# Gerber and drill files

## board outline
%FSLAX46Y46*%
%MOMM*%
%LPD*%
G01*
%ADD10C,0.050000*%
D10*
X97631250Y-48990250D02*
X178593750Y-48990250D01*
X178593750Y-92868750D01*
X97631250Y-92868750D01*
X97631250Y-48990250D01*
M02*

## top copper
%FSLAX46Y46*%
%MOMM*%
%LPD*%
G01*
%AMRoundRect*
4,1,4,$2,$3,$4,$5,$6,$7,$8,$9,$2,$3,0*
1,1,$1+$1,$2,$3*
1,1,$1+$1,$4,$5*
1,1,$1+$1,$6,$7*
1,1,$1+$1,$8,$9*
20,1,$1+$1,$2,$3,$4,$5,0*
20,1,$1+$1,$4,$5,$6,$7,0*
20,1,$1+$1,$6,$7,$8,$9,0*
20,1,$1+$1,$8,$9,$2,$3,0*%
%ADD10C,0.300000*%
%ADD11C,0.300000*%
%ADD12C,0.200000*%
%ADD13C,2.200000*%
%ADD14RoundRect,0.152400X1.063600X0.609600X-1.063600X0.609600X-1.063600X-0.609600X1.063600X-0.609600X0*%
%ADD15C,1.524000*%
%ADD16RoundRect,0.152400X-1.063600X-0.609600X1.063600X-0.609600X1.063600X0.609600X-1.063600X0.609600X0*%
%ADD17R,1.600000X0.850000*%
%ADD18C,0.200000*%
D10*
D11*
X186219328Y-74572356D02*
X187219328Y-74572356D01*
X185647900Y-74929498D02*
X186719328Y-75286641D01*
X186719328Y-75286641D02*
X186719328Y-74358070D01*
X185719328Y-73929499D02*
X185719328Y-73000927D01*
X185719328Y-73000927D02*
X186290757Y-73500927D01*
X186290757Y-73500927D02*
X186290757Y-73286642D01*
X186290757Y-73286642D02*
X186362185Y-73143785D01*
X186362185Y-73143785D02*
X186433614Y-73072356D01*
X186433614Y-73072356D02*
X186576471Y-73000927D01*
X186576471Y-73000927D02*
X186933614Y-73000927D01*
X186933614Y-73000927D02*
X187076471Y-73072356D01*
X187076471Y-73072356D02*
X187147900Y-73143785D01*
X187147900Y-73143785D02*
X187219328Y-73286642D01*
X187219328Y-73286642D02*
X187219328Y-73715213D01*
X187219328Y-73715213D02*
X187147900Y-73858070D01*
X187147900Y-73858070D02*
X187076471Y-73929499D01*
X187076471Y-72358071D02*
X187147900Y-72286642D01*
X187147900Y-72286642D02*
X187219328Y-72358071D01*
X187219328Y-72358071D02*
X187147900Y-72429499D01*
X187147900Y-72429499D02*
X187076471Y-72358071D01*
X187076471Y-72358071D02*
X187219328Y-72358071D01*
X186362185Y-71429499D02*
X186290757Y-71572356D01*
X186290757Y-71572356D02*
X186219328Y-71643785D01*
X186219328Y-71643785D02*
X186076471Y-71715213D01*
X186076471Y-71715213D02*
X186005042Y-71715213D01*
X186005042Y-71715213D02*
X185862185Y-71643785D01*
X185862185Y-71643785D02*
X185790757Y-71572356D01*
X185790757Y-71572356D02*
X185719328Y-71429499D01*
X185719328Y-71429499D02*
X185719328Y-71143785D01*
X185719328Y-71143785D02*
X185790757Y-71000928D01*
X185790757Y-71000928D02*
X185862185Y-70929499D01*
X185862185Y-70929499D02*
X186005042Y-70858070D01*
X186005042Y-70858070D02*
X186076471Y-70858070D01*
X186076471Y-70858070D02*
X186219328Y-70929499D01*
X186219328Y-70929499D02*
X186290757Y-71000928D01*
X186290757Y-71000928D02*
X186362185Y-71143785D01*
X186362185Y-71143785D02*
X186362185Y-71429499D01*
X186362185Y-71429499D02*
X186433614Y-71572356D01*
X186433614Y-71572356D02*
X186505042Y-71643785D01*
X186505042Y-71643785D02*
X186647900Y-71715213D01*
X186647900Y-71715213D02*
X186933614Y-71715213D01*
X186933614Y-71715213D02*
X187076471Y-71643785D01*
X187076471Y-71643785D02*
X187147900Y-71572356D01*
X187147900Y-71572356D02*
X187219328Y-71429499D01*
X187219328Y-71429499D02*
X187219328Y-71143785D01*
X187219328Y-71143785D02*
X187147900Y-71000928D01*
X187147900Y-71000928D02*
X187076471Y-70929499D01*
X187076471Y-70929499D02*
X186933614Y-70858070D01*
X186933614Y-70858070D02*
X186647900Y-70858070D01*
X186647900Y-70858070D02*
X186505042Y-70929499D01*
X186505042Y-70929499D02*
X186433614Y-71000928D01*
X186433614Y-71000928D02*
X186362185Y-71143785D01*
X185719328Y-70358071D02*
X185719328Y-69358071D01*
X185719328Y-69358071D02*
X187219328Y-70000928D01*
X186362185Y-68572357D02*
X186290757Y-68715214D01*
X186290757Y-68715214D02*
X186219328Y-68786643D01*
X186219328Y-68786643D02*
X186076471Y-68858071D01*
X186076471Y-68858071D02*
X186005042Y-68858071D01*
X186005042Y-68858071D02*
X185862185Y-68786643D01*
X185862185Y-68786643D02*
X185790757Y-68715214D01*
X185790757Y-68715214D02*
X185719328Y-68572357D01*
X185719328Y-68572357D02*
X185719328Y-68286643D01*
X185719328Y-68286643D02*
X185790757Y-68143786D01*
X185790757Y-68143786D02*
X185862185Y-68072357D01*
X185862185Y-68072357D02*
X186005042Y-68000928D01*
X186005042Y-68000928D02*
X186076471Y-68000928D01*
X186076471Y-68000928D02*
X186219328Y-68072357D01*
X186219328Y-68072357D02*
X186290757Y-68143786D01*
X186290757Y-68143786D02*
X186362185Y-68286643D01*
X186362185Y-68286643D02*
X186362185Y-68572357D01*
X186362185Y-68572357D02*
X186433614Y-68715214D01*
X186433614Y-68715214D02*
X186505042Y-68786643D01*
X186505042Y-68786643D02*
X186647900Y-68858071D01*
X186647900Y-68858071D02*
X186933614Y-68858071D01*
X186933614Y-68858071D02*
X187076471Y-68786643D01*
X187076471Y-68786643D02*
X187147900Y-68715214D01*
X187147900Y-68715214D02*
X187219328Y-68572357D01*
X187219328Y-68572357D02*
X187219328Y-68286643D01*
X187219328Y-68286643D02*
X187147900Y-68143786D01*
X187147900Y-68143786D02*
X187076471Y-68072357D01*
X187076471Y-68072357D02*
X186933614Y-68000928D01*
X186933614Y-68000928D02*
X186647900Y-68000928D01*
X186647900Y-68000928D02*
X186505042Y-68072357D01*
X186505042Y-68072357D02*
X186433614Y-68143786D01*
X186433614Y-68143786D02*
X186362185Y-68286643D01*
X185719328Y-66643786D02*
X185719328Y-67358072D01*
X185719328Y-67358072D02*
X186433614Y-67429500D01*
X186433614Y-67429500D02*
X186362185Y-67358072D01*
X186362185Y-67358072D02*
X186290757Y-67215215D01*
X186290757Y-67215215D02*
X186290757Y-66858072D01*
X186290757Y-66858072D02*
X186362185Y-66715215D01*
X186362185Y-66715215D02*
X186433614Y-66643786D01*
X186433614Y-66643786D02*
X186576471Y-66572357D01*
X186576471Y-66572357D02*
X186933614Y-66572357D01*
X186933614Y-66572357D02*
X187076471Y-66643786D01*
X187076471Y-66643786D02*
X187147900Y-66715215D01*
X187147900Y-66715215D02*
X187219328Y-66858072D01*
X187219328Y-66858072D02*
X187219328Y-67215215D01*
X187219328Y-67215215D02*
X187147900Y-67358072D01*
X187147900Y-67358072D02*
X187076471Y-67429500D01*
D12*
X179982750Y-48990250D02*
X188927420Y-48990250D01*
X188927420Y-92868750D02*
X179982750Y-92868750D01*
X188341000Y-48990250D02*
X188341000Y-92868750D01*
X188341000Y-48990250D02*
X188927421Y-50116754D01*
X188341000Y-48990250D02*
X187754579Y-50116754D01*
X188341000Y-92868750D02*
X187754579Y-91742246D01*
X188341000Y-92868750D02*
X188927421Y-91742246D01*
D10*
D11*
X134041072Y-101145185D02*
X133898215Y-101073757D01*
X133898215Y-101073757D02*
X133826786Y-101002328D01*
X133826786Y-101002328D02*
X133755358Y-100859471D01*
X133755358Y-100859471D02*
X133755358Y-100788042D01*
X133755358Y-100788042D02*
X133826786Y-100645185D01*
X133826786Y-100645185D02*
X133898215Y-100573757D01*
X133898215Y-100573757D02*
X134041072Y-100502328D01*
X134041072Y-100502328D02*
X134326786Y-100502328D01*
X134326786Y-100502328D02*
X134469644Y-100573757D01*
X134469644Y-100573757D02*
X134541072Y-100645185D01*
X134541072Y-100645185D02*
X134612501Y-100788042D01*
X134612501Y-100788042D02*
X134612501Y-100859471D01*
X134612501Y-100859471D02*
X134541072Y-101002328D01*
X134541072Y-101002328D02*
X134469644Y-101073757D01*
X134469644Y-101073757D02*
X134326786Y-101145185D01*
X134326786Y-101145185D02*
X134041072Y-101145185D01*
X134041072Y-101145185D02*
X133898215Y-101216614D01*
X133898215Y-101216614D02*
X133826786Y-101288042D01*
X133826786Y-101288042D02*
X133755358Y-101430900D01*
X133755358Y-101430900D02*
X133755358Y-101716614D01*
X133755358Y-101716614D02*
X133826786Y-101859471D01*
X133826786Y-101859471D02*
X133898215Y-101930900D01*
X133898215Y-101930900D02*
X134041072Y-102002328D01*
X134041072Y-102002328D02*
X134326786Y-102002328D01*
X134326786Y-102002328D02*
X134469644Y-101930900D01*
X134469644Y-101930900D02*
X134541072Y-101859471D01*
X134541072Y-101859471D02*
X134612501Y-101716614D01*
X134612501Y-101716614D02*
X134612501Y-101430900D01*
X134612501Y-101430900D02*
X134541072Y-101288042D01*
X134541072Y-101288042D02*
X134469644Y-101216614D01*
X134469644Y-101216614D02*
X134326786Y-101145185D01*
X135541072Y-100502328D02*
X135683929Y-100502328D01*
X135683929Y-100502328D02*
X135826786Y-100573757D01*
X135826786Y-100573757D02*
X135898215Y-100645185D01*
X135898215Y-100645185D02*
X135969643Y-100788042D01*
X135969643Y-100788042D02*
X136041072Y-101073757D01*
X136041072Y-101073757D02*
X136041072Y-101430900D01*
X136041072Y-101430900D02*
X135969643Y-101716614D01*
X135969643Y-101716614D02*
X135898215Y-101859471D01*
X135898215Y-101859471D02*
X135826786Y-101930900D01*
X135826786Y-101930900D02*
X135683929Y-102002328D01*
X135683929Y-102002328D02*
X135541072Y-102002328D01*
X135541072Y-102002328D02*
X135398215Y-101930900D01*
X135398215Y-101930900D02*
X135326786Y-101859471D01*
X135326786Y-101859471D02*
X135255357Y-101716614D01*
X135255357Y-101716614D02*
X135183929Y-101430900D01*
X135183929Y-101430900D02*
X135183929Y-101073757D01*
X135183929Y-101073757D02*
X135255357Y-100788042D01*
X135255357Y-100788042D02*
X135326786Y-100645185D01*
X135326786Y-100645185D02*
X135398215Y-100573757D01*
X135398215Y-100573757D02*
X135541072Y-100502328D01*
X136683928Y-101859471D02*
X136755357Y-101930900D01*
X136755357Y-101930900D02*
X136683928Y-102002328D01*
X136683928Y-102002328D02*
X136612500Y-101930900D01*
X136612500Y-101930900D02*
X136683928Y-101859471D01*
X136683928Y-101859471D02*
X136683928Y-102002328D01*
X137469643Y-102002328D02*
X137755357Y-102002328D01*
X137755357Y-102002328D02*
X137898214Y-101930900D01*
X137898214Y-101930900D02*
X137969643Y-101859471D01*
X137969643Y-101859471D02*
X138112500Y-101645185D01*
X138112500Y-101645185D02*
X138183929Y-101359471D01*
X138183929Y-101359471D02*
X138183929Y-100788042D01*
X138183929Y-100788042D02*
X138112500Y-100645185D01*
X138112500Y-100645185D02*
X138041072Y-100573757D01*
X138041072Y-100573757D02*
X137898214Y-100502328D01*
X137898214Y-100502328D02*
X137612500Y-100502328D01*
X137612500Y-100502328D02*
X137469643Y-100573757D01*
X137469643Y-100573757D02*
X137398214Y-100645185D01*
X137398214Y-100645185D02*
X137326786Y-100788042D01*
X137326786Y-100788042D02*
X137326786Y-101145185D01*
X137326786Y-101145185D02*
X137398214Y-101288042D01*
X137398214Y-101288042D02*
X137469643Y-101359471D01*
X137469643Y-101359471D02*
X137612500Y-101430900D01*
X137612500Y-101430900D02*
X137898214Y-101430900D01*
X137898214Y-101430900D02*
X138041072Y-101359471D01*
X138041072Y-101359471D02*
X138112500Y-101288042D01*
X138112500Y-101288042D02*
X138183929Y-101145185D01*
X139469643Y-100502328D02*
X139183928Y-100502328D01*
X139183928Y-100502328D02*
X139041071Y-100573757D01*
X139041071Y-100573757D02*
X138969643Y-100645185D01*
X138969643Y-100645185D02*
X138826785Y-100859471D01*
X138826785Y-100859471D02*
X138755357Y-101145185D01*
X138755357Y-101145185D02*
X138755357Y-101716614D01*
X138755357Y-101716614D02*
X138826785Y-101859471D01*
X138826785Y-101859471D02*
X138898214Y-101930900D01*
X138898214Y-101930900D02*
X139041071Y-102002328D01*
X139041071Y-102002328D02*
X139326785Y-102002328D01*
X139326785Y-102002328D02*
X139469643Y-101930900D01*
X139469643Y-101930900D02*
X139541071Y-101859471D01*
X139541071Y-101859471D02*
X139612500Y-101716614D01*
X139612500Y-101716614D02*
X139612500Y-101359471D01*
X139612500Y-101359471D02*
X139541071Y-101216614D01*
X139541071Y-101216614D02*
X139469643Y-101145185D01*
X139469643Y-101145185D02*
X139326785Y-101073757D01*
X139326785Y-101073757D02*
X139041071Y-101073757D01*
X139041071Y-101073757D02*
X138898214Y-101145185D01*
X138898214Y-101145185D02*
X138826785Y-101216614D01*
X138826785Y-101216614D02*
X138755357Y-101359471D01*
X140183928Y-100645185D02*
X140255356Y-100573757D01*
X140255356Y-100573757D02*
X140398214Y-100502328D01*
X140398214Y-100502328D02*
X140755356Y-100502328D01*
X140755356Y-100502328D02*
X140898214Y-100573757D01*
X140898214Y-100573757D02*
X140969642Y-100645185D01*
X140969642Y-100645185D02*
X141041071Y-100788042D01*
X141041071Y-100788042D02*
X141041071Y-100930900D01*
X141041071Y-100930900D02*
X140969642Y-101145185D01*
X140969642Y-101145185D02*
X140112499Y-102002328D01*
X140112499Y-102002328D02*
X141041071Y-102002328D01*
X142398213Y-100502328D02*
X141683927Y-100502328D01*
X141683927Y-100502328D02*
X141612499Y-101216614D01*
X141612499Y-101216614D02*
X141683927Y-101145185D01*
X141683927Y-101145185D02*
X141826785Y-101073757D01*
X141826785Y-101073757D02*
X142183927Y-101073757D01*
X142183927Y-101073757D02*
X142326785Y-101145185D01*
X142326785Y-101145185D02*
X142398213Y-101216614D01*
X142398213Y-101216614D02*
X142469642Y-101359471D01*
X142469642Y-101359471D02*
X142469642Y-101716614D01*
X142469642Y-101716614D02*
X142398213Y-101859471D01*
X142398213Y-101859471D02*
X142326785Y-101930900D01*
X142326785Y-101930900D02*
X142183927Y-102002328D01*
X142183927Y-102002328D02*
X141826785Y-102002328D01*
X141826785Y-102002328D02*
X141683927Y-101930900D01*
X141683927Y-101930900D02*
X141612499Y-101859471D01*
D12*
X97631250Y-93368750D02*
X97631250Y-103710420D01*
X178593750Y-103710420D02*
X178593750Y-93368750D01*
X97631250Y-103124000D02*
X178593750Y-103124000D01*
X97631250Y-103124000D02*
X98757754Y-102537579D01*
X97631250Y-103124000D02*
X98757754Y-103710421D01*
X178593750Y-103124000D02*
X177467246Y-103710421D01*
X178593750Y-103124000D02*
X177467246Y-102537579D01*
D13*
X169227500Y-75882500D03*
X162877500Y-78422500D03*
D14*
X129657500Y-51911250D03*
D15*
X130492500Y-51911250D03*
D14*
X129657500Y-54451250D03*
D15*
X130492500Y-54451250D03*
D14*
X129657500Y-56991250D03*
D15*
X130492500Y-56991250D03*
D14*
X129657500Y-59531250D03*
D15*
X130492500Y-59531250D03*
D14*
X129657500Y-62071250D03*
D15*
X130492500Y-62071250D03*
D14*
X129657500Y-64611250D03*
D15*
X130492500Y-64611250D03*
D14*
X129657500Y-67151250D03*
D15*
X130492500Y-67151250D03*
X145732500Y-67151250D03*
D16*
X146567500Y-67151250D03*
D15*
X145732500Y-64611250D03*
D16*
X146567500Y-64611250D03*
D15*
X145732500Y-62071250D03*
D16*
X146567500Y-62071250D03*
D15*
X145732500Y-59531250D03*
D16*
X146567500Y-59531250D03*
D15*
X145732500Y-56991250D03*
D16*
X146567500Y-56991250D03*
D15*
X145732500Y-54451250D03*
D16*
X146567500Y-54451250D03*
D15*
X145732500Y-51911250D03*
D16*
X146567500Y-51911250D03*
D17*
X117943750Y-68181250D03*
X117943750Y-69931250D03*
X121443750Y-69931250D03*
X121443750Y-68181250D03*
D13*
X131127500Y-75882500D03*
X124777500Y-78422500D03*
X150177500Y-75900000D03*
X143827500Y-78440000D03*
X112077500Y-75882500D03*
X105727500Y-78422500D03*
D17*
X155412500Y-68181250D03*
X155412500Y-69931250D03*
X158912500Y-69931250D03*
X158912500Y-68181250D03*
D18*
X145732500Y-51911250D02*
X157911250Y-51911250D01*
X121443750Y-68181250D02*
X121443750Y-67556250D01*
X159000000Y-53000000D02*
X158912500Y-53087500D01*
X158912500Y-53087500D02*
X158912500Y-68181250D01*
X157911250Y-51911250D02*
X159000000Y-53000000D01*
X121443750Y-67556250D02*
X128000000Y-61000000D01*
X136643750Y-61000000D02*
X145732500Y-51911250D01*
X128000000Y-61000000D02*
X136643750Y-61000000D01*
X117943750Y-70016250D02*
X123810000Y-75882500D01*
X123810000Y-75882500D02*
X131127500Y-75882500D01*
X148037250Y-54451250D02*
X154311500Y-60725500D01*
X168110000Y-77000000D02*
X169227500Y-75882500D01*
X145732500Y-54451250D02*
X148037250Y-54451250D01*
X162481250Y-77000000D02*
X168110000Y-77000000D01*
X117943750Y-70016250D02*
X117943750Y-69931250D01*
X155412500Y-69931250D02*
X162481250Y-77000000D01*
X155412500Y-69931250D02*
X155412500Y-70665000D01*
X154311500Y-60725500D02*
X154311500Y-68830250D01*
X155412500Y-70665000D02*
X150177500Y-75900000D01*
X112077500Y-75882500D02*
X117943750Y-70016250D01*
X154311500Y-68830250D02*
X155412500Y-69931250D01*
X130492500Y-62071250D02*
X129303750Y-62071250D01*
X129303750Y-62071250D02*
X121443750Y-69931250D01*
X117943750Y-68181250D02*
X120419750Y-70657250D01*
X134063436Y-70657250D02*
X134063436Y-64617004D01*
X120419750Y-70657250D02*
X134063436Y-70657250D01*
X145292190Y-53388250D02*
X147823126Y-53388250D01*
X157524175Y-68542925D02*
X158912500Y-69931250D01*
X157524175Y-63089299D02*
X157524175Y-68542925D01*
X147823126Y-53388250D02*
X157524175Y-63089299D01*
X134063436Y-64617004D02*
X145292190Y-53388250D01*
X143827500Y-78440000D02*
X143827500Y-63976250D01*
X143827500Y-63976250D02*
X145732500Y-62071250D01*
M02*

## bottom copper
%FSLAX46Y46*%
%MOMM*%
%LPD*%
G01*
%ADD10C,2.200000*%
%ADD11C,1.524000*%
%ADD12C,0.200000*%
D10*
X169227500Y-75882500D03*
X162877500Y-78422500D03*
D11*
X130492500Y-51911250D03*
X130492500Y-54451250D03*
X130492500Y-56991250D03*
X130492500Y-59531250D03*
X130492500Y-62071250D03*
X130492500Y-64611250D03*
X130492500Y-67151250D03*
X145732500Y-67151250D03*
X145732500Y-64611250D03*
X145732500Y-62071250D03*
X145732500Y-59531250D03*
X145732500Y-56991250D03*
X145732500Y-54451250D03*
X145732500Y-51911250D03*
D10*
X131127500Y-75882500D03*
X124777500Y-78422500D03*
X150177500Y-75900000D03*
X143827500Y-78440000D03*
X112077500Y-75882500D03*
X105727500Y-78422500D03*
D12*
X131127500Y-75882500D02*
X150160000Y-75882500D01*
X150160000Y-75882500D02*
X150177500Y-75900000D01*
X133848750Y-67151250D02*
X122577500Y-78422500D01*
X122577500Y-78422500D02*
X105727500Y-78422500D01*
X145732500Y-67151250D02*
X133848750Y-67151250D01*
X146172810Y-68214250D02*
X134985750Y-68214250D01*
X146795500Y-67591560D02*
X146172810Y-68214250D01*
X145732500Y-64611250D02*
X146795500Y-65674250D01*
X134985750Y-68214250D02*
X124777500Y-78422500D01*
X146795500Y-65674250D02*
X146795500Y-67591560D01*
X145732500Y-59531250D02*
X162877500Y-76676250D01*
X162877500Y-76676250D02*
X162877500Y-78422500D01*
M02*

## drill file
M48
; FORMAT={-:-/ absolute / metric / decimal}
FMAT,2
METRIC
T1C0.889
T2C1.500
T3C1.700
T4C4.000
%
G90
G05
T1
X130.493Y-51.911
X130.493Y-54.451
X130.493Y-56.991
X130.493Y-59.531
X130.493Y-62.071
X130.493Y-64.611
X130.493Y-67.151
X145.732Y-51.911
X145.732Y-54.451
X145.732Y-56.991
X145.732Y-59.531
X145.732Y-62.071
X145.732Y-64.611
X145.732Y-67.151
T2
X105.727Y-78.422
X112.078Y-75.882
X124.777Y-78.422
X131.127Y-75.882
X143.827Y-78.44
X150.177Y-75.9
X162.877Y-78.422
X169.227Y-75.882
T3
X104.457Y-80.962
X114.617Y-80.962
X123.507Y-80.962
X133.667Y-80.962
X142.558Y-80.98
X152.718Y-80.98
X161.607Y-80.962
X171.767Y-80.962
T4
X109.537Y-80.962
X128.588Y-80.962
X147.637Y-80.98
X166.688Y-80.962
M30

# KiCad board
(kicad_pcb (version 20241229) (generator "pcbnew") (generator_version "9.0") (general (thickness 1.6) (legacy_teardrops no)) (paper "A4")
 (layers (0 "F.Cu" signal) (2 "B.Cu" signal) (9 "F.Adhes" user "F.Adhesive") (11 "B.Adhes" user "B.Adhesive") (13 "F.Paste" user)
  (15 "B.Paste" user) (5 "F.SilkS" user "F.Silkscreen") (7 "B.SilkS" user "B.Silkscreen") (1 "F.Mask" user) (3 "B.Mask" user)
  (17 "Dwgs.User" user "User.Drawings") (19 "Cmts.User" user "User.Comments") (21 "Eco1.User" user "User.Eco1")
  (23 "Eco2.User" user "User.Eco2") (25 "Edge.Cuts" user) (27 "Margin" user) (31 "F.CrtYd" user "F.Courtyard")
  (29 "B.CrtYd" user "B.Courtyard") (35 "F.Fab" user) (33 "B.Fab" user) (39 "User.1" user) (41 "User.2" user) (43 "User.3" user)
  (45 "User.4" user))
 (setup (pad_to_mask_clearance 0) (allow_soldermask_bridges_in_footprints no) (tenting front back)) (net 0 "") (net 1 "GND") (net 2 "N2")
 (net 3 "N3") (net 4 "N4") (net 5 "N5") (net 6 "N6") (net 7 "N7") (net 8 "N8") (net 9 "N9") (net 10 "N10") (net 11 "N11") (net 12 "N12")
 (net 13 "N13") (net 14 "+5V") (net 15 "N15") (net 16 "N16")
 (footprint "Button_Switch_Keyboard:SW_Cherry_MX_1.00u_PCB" (layer "F.Cu") (at 169.2275 75.8825)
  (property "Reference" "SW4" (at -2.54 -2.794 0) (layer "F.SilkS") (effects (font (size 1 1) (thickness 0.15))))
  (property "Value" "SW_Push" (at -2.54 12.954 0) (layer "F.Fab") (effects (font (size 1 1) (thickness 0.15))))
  (pad "" np_thru_hole circle (at -7.62 5.08) (size 1.7 1.7) (drill 1.7) (layers "*.Cu" "*.Mask"))
  (pad "" np_thru_hole circle (at -2.54 5.08) (size 4 4) (drill 4) (layers "*.Cu" "*.Mask"))
  (pad "" np_thru_hole circle (at 2.54 5.08) (size 1.7 1.7) (drill 1.7) (layers "*.Cu" "*.Mask"))
  (pad "1" thru_hole circle (at 0 0) (size 2.2 2.2) (drill 1.5) (layers "*.Cu" "*.Mask") (remove_unused_layers no) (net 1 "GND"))
  (pad "2" thru_hole circle (at -6.35 2.54) (size 2.2 2.2) (drill 1.5) (layers "*.Cu" "*.Mask") (remove_unused_layers no) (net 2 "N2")))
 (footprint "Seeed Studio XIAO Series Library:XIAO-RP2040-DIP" (layer "F.Cu") (at 138.1125 59.53125)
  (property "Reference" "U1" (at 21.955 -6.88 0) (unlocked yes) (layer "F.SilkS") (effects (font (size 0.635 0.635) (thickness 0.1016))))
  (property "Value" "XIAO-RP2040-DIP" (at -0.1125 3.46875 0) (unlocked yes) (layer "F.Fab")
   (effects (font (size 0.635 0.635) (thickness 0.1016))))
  (pad "1" smd roundrect (at -8.455 -7.62 180) (size 2.432 1.524) (layers "F.Cu" "F.Mask") (roundrect_rratio 0.1) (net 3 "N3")
   (thermal_bridge_angle 45))
  (pad "1" thru_hole circle (at -7.62 -7.62 180) (size 1.524 1.524) (drill 0.889) (layers "*.Cu" "*.Mask") (remove_unused_layers no)
   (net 3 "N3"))
  (pad "2" smd roundrect (at -8.455 -5.08 180) (size 2.432 1.524) (layers "F.Cu" "F.Mask") (roundrect_rratio 0.1) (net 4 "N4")
   (thermal_bridge_angle 45))
  (pad "2" thru_hole circle (at -7.62 -5.08 180) (size 1.524 1.524) (drill 0.889) (layers "*.Cu" "*.Mask") (remove_unused_layers no)
   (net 4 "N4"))
  (pad "3" smd roundrect (at -8.455 -2.54 180) (size 2.432 1.524) (layers "F.Cu" "F.Mask") (roundrect_rratio 0.1) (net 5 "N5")
   (thermal_bridge_angle 45))
  (pad "3" thru_hole circle (at -7.62 -2.54 180) (size 1.524 1.524) (drill 0.889) (layers "*.Cu" "*.Mask") (remove_unused_layers no)
   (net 5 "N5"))
  (pad "4" smd roundrect (at -8.455 0 180) (size 2.432 1.524) (layers "F.Cu" "F.Mask") (roundrect_rratio 0.1) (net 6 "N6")
   (thermal_bridge_angle 45))
  (pad "4" thru_hole circle (at -7.62 0 180) (size 1.524 1.524) (drill 0.889) (layers "*.Cu" "*.Mask") (remove_unused_layers no)
   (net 6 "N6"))
  (pad "5" smd roundrect (at -8.455 2.54 180) (size 2.432 1.524) (layers "F.Cu" "F.Mask") (roundrect_rratio 0.1) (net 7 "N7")
   (thermal_bridge_angle 45))
  (pad "5" thru_hole circle (at -7.62 2.54 180) (size 1.524 1.524) (drill 0.889) (layers "*.Cu" "*.Mask") (remove_unused_layers no)
   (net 7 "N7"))
  (pad "6" smd roundrect (at -8.455 5.08 180) (size 2.432 1.524) (layers "F.Cu" "F.Mask") (roundrect_rratio 0.1) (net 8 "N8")
   (thermal_bridge_angle 45))
  (pad "6" thru_hole circle (at -7.62 5.08 180) (size 1.524 1.524) (drill 0.889) (layers "*.Cu" "*.Mask") (remove_unused_layers no)
   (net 8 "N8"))
  (pad "7" smd roundrect (at -8.455 7.62 180) (size 2.432 1.524) (layers "F.Cu" "F.Mask") (roundrect_rratio 0.1) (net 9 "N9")
   (thermal_bridge_angle 45))
  (pad "7" thru_hole circle (at -7.62 7.62 180) (size 1.524 1.524) (drill 0.889) (layers "*.Cu" "*.Mask") (remove_unused_layers no)
   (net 9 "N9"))
  (pad "8" thru_hole circle (at 7.62 7.62) (size 1.524 1.524) (drill 0.889) (layers "*.Cu" "*.Mask") (remove_unused_layers no)
   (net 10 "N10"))
  (pad "8" smd roundrect (at 8.455 7.62) (size 2.432 1.524) (layers "F.Cu" "F.Mask") (roundrect_rratio 0.1) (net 10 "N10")
   (thermal_bridge_angle 45))
  (pad "9" thru_hole circle (at 7.62 5.08) (size 1.524 1.524) (drill 0.889) (layers "*.Cu" "*.Mask") (remove_unused_layers no)
   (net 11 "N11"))
  (pad "9" smd roundrect (at 8.455 5.08) (size 2.432 1.524) (layers "F.Cu" "F.Mask") (roundrect_rratio 0.1) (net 11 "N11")
   (thermal_bridge_angle 45))
  (pad "10" thru_hole circle (at 7.62 2.54) (size 1.524 1.524) (drill 0.889) (layers "*.Cu" "*.Mask") (remove_unused_layers no)
   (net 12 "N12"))
  (pad "10" smd roundrect (at 8.455 2.54) (size 2.432 1.524) (layers "F.Cu" "F.Mask") (roundrect_rratio 0.1) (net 12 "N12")
   (thermal_bridge_angle 45))
  (pad "11" thru_hole circle (at 7.62 0) (size 1.524 1.524) (drill 0.889) (layers "*.Cu" "*.Mask") (remove_unused_layers no) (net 2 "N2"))
  (pad "11" smd roundrect (at 8.455 0) (size 2.432 1.524) (layers "F.Cu" "F.Mask") (roundrect_rratio 0.1) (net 2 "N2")
   (thermal_bridge_angle 45))
  (pad "12" thru_hole circle (at 7.62 -2.54) (size 1.524 1.524) (drill 0.889) (layers "*.Cu" "*.Mask") (remove_unused_layers no)
   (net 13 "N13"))
  (pad "12" smd roundrect (at 8.455 -2.54) (size 2.432 1.524) (layers "F.Cu" "F.Mask") (roundrect_rratio 0.1) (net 13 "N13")
   (thermal_bridge_angle 45))
  (pad "13" thru_hole circle (at 7.62 -5.08) (size 1.524 1.524) (drill 0.889) (layers "*.Cu" "*.Mask") (remove_unused_layers no)
   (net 1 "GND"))
  (pad "13" smd roundrect (at 8.455 -5.08) (size 2.432 1.524) (layers "F.Cu" "F.Mask") (roundrect_rratio 0.1) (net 1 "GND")
   (thermal_bridge_angle 45))
  (pad "14" thru_hole circle (at 7.62 -7.62) (size 1.524 1.524) (drill 0.889) (layers "*.Cu" "*.Mask") (remove_unused_layers no)
   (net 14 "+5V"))
  (pad "14" smd roundrect (at 8.455 -7.62) (size 2.432 1.524) (layers "F.Cu" "F.Mask") (roundrect_rratio 0.1) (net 14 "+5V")
   (thermal_bridge_angle 45)))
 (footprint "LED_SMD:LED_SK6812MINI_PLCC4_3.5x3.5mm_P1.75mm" (layer "F.Cu") (at 119.69375 69.05625)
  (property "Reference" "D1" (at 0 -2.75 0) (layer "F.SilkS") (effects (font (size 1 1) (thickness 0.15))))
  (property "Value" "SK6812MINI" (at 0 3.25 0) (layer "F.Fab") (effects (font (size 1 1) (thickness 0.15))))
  (pad "1" smd rect (at -1.75 -0.875) (size 1.6 0.85) (layers "F.Cu" "F.Mask" "F.Paste") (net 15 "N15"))
  (pad "2" smd rect (at -1.75 0.875) (size 1.6 0.85) (layers "F.Cu" "F.Mask" "F.Paste") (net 1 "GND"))
  (pad "3" smd rect (at 1.75 0.875) (size 1.6 0.85) (layers "F.Cu" "F.Mask" "F.Paste") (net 7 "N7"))
  (pad "4" smd rect (at 1.75 -0.875) (size 1.6 0.85) (layers "F.Cu" "F.Mask" "F.Paste") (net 14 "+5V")))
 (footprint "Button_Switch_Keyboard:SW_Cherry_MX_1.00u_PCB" (layer "F.Cu") (at 131.1275 75.8825)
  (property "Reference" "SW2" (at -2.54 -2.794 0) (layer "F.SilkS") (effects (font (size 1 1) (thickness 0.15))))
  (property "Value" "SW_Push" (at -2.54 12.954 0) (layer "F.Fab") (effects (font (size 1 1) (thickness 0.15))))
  (pad "" np_thru_hole circle (at -7.62 5.08) (size 1.7 1.7) (drill 1.7) (layers "*.Cu" "*.Mask"))
  (pad "" np_thru_hole circle (at -2.54 5.08) (size 4 4) (drill 4) (layers "*.Cu" "*.Mask"))
  (pad "" np_thru_hole circle (at 2.54 5.08) (size 1.7 1.7) (drill 1.7) (layers "*.Cu" "*.Mask"))
  (pad "1" thru_hole circle (at 0 0) (size 2.2 2.2) (drill 1.5) (layers "*.Cu" "*.Mask") (remove_unused_layers no) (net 1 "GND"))
  (pad "2" thru_hole circle (at -6.35 2.54) (size 2.2 2.2) (drill 1.5) (layers "*.Cu" "*.Mask") (remove_unused_layers no) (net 11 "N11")))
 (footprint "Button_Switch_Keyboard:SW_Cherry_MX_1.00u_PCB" (layer "F.Cu") (at 150.1775 75.9)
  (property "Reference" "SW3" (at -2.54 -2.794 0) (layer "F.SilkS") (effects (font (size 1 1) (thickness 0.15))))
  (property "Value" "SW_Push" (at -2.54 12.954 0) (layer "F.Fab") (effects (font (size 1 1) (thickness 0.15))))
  (pad "" np_thru_hole circle (at -7.62 5.08) (size 1.7 1.7) (drill 1.7) (layers "*.Cu" "*.Mask"))
  (pad "" np_thru_hole circle (at -2.54 5.08) (size 4 4) (drill 4) (layers "*.Cu" "*.Mask"))
  (pad "" np_thru_hole circle (at 2.54 5.08) (size 1.7 1.7) (drill 1.7) (layers "*.Cu" "*.Mask"))
  (pad "1" thru_hole circle (at 0 0) (size 2.2 2.2) (drill 1.5) (layers "*.Cu" "*.Mask") (remove_unused_layers no) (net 1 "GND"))
  (pad "2" thru_hole circle (at -6.35 2.54) (size 2.2 2.2) (drill 1.5) (layers "*.Cu" "*.Mask") (remove_unused_layers no) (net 12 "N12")))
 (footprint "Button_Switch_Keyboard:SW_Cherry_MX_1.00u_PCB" (layer "F.Cu") (at 112.0775 75.8825)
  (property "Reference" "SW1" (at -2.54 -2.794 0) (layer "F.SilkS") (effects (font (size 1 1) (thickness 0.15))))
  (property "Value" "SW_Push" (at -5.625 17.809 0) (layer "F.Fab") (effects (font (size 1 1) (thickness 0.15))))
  (pad "" np_thru_hole circle (at -7.62 5.08) (size 1.7 1.7) (drill 1.7) (layers "*.Cu" "*.Mask"))
  (pad "" np_thru_hole circle (at -2.54 5.08) (size 4 4) (drill 4) (layers "*.Cu" "*.Mask"))
  (pad "" np_thru_hole circle (at 2.54 5.08) (size 1.7 1.7) (drill 1.7) (layers "*.Cu" "*.Mask"))
  (pad "1" thru_hole circle (at 0 0) (size 2.2 2.2) (drill 1.5) (layers "*.Cu" "*.Mask") (remove_unused_layers no) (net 1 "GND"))
  (pad "2" thru_hole circle (at -6.35 2.54) (size 2.2 2.2) (drill 1.5) (layers "*.Cu" "*.Mask") (remove_unused_layers no) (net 10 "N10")))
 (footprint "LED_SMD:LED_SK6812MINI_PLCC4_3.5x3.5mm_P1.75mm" (layer "F.Cu") (at 157.1625 69.05625)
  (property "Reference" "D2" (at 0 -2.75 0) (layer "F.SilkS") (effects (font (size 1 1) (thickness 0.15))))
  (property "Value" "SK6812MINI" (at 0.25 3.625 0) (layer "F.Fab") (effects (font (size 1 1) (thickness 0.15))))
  (pad "1" smd rect (at -1.75 -0.875) (size 1.6 0.85) (layers "F.Cu" "F.Mask" "F.Paste") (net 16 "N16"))
  (pad "2" smd rect (at -1.75 0.875) (size 1.6 0.85) (layers "F.Cu" "F.Mask" "F.Paste") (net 1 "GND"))
  (pad "3" smd rect (at 1.75 0.875) (size 1.6 0.85) (layers "F.Cu" "F.Mask" "F.Paste") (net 15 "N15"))
  (pad "4" smd rect (at 1.75 -0.875) (size 1.6 0.85) (layers "F.Cu" "F.Mask" "F.Paste") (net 14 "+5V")))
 (gr_rect (start 97.63125 48.99025) (end 178.59375 92.86875) (stroke (width 0.05) (type default)) (fill no) (layer "Edge.Cuts"))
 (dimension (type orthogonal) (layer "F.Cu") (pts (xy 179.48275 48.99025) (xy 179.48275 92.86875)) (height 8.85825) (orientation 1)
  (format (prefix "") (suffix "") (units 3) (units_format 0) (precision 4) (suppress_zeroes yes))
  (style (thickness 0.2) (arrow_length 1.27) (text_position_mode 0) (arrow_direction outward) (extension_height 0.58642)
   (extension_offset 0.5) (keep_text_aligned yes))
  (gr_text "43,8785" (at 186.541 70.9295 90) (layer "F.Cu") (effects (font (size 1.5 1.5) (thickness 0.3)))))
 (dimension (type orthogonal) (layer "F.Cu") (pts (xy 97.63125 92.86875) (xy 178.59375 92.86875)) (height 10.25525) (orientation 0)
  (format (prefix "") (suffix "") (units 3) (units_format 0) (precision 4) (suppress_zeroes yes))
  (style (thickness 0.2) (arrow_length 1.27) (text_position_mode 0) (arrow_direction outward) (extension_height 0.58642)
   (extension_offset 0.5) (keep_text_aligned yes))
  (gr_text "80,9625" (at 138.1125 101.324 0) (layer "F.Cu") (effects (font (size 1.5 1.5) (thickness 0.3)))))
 (segment (start 145.7325 51.91125) (end 157.91125 51.91125) (width 0.2) (layer "F.Cu") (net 14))
 (segment (start 121.44375 68.18125) (end 121.44375 67.55625) (width 0.2) (layer "F.Cu") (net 14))
 (segment (start 159 53) (end 158.9125 53.0875) (width 0.2) (layer "F.Cu") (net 14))
 (segment (start 158.9125 53.0875) (end 158.9125 68.18125) (width 0.2) (layer "F.Cu") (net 14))
 (segment (start 157.91125 51.91125) (end 159 53) (width 0.2) (layer "F.Cu") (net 14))
 (segment (start 121.44375 67.55625) (end 128 61) (width 0.2) (layer "F.Cu") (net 14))
 (segment (start 136.64375 61) (end 145.7325 51.91125) (width 0.2) (layer "F.Cu") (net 14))
 (segment (start 128 61) (end 136.64375 61) (width 0.2) (layer "F.Cu") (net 14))
 (segment (start 117.94375 70.01625) (end 123.81 75.8825) (width 0.2) (layer "F.Cu") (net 1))
 (segment (start 123.81 75.8825) (end 131.1275 75.8825) (width 0.2) (layer "F.Cu") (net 1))
 (segment (start 148.03725 54.45125) (end 154.3115 60.7255) (width 0.2) (layer "F.Cu") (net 1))
 (segment (start 168.11 77) (end 169.2275 75.8825) (width 0.2) (layer "F.Cu") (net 1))
 (segment (start 145.7325 54.45125) (end 148.03725 54.45125) (width 0.2) (layer "F.Cu") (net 1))
 (segment (start 162.48125 77) (end 168.11 77) (width 0.2) (layer "F.Cu") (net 1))
 (segment (start 117.94375 70.01625) (end 117.94375 69.93125) (width 0.2) (layer "F.Cu") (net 1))
 (segment (start 155.4125 69.93125) (end 162.48125 77) (width 0.2) (layer "F.Cu") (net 1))
 (segment (start 155.4125 69.93125) (end 155.4125 70.665) (width 0.2) (layer "F.Cu") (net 1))
 (segment (start 154.3115 60.7255) (end 154.3115 68.83025) (width 0.2) (layer "F.Cu") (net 1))
 (segment (start 155.4125 70.665) (end 150.1775 75.9) (width 0.2) (layer "F.Cu") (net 1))
 (segment (start 112.0775 75.8825) (end 117.94375 70.01625) (width 0.2) (layer "F.Cu") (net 1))
 (segment (start 154.3115 68.83025) (end 155.4125 69.93125) (width 0.2) (layer "F.Cu") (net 1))
 (segment (start 131.1275 75.8825) (end 150.16 75.8825) (width 0.2) (layer "B.Cu") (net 1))
 (segment (start 150.16 75.8825) (end 150.1775 75.9) (width 0.2) (layer "B.Cu") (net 1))
 (segment (start 130.4925 62.07125) (end 129.30375 62.07125) (width 0.2) (layer "F.Cu") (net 7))
 (segment (start 129.30375 62.07125) (end 121.44375 69.93125) (width 0.2) (layer "F.Cu") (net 7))
 (segment (start 117.94375 68.18125) (end 120.41975 70.65725) (width 0.2) (layer "F.Cu") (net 15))
 (segment (start 134.063436 70.65725) (end 134.063436 64.617004) (width 0.2) (layer "F.Cu") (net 15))
 (segment (start 120.41975 70.65725) (end 134.063436 70.65725) (width 0.2) (layer "F.Cu") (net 15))
 (segment (start 145.29219 53.38825) (end 147.823126 53.38825) (width 0.2) (layer "F.Cu") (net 15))
 (segment (start 157.524175 68.542925) (end 158.9125 69.93125) (width 0.2) (layer "F.Cu") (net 15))
 (segment (start 157.524175 63.089299) (end 157.524175 68.542925) (width 0.2) (layer "F.Cu") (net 15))
 (segment (start 147.823126 53.38825) (end 157.524175 63.089299) (width 0.2) (layer "F.Cu") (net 15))
 (segment (start 134.063436 64.617004) (end 145.29219 53.38825) (width 0.2) (layer "F.Cu") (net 15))
 (segment (start 133.84875 67.15125) (end 122.5775 78.4225) (width 0.2) (layer "B.Cu") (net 10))
 (segment (start 122.5775 78.4225) (end 105.7275 78.4225) (width 0.2) (layer "B.Cu") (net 10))
 (segment (start 145.7325 67.15125) (end 133.84875 67.15125) (width 0.2) (layer "B.Cu") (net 10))
 (segment (start 146.17281 68.21425) (end 134.98575 68.21425) (width 0.2) (layer "B.Cu") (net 11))
 (segment (start 146.7955 67.59156) (end 146.17281 68.21425) (width 0.2) (layer "B.Cu") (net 11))
 (segment (start 145.7325 64.61125) (end 146.7955 65.67425) (width 0.2) (layer "B.Cu") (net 11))
 (segment (start 134.98575 68.21425) (end 124.7775 78.4225) (width 0.2) (layer "B.Cu") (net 11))
 (segment (start 146.7955 65.67425) (end 146.7955 67.59156) (width 0.2) (layer "B.Cu") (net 11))
 (segment (start 143.8275 78.44) (end 143.8275 63.97625) (width 0.2) (layer "F.Cu") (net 12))
 (segment (start 143.8275 63.97625) (end 145.7325 62.07125) (width 0.2) (layer "F.Cu") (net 12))
 (segment (start 145.7325 59.53125) (end 162.8775 76.67625) (width 0.2) (layer "B.Cu") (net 2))
 (segment (start 162.8775 76.67625) (end 162.8775 78.4225) (width 0.2) (layer "B.Cu") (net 2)))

